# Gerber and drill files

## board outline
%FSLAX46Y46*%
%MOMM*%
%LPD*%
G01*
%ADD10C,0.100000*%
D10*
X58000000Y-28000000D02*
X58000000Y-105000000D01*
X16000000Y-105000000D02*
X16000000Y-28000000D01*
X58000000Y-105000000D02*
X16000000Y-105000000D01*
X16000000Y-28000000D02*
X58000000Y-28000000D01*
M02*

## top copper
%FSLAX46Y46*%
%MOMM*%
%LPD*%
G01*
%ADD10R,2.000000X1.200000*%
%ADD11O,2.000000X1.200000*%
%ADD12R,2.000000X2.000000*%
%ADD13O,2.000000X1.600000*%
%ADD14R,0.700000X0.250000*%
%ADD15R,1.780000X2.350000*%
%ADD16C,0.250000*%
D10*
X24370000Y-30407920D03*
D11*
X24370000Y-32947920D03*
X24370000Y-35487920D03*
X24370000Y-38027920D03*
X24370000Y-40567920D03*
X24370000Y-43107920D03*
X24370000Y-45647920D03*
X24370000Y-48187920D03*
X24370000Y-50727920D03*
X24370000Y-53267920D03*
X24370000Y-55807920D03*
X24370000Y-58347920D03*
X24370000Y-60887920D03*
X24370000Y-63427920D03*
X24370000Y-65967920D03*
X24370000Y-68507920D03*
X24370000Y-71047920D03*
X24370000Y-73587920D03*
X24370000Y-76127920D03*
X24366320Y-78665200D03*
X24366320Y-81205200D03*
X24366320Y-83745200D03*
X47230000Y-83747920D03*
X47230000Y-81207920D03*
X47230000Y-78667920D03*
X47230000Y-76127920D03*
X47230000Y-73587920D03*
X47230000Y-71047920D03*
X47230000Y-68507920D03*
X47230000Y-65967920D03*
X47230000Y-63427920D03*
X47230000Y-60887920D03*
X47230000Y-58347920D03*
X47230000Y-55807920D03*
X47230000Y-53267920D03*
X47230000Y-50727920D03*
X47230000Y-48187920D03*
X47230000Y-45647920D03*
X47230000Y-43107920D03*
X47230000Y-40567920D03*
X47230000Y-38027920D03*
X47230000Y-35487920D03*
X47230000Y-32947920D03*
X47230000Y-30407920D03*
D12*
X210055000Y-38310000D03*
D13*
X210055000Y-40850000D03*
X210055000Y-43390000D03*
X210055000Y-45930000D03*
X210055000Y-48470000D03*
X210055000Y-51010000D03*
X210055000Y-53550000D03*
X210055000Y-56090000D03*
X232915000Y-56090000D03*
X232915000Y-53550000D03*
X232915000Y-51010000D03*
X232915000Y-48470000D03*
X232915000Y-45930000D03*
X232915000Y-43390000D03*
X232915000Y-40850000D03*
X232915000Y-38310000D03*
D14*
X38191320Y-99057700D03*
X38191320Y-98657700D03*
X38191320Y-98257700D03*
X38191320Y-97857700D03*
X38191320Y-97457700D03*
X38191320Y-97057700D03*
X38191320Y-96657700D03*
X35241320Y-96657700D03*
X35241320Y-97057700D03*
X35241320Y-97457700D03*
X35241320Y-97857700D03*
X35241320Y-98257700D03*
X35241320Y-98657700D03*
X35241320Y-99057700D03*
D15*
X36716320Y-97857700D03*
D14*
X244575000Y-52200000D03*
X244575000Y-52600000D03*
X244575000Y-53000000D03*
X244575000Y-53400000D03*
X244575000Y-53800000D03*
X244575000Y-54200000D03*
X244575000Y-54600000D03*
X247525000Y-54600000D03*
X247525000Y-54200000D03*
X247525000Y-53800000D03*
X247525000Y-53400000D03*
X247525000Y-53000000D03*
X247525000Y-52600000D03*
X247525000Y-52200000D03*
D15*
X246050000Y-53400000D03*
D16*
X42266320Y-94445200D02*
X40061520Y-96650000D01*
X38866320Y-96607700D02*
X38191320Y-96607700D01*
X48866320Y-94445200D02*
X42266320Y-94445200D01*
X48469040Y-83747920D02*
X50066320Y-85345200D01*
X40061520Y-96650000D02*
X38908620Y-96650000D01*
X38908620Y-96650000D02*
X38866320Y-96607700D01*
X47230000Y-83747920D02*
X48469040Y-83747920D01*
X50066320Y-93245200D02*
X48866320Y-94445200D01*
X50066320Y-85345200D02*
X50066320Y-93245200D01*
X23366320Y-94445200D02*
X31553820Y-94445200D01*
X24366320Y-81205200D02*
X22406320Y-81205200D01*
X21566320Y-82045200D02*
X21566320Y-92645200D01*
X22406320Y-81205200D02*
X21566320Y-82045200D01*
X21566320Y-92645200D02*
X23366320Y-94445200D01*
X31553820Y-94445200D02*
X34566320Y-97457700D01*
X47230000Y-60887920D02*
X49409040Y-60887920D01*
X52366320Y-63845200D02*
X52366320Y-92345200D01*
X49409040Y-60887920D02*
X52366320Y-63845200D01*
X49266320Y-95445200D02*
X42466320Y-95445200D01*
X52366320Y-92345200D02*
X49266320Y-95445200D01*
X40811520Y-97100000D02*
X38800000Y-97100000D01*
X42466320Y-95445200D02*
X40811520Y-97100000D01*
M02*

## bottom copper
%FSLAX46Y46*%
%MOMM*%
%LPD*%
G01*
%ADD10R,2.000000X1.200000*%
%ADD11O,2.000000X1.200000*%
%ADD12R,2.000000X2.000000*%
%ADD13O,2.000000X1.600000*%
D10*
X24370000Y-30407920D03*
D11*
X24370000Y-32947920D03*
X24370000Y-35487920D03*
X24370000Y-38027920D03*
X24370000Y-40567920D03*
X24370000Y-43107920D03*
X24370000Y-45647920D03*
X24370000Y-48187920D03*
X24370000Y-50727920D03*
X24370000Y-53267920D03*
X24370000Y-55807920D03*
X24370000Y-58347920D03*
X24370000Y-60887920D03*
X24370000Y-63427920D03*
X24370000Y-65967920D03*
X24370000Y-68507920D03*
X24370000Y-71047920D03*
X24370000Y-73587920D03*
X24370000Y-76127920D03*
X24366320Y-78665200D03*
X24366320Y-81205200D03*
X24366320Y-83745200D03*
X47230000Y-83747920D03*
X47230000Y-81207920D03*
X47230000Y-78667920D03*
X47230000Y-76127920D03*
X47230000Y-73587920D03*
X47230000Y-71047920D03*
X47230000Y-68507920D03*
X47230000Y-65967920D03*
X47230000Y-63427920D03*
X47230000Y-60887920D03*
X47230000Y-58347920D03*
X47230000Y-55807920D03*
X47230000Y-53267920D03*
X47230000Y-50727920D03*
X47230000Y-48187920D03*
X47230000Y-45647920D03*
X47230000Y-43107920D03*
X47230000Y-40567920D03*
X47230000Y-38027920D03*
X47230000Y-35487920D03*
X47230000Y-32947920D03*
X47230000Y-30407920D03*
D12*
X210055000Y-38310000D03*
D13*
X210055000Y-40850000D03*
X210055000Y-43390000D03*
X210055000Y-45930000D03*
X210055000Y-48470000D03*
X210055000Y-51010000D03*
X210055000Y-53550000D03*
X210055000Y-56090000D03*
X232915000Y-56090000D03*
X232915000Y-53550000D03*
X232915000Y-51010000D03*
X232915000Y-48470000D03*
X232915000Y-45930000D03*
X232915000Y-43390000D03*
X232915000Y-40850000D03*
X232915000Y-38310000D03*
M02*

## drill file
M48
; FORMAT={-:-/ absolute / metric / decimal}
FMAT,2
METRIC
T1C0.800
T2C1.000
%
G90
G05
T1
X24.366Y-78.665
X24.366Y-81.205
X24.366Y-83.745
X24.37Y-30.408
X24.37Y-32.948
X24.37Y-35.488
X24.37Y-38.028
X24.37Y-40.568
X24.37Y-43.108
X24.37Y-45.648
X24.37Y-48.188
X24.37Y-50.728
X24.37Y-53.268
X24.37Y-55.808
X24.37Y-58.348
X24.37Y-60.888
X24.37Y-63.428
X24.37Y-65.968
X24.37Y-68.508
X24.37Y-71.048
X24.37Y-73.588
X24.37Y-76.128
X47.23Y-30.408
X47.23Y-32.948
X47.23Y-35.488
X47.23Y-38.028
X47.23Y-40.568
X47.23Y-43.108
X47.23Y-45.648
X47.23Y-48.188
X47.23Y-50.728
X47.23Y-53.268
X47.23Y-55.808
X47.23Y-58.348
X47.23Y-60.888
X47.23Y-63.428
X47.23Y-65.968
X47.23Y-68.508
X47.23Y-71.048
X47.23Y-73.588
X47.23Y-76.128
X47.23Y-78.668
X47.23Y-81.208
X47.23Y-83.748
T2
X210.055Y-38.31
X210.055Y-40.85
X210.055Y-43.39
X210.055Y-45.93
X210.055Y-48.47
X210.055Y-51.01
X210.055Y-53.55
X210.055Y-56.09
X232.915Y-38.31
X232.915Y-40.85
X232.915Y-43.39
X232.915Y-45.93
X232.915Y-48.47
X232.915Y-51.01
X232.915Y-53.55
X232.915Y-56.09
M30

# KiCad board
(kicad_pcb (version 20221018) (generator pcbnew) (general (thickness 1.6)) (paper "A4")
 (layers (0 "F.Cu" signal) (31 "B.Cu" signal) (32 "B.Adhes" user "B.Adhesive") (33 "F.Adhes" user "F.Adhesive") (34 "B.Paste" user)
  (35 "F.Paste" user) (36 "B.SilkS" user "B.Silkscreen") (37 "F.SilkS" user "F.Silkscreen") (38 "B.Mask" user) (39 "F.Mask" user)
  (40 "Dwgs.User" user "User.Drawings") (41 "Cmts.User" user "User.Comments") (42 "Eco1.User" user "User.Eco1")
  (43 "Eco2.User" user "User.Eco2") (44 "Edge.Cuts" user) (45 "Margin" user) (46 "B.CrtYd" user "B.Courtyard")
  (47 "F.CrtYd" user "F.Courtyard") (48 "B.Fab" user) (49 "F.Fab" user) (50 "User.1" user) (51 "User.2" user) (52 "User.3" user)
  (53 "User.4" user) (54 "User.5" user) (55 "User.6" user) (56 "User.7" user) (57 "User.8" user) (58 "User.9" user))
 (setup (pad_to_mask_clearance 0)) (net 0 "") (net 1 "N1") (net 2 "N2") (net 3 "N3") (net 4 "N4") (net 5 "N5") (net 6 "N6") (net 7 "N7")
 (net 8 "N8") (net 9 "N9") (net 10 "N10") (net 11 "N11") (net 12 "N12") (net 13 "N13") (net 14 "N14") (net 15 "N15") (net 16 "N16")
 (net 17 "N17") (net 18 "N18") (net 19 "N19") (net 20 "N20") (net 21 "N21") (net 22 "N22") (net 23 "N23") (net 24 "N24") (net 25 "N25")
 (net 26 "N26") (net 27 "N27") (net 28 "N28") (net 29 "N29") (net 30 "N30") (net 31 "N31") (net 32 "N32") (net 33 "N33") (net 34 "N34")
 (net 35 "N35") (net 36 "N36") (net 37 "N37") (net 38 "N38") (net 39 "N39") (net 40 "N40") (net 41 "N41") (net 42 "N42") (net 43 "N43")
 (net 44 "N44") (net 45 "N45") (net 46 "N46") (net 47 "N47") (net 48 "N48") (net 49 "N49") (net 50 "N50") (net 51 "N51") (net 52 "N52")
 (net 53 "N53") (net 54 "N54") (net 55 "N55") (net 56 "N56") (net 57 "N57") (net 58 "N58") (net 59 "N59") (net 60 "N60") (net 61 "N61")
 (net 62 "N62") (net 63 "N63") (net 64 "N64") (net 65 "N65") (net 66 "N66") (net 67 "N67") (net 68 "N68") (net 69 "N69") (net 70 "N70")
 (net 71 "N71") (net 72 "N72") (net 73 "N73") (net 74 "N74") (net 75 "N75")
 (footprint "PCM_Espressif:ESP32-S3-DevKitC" (layer "F.Cu") (at 24.37 30.40792)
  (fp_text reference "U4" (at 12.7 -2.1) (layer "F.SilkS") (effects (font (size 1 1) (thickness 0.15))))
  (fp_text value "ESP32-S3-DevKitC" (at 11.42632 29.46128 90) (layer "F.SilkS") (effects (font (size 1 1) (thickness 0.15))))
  (pad "1" thru_hole rect (at 0 0 270) (size 1.2 2) (drill 0.8) (layers "*.Cu" "*.Mask") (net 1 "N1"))
  (pad "2" thru_hole oval (at 0 2.54 270) (size 1.2 2) (drill 0.8) (layers "*.Cu" "*.Mask") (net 1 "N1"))
  (pad "3" thru_hole oval (at 0 5.08 270) (size 1.2 2) (drill 0.8) (layers "*.Cu" "*.Mask") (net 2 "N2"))
  (pad "4" thru_hole oval (at 0 7.62 270) (size 1.2 2) (drill 0.8) (layers "*.Cu" "*.Mask") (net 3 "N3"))
  (pad "5" thru_hole oval (at 0 10.16 270) (size 1.2 2) (drill 0.8) (layers "*.Cu" "*.Mask") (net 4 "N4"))
  (pad "6" thru_hole oval (at 0 12.7 270) (size 1.2 2) (drill 0.8) (layers "*.Cu" "*.Mask") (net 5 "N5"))
  (pad "7" thru_hole oval (at 0 15.24 270) (size 1.2 2) (drill 0.8) (layers "*.Cu" "*.Mask") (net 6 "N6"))
  (pad "8" thru_hole oval (at 0 17.78 270) (size 1.2 2) (drill 0.8) (layers "*.Cu" "*.Mask") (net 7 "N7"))
  (pad "9" thru_hole oval (at 0 20.32 270) (size 1.2 2) (drill 0.8) (layers "*.Cu" "*.Mask") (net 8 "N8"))
  (pad "10" thru_hole oval (at 0 22.86 270) (size 1.2 2) (drill 0.8) (layers "*.Cu" "*.Mask") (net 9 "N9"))
  (pad "11" thru_hole oval (at 0 25.4 270) (size 1.2 2) (drill 0.8) (layers "*.Cu" "*.Mask") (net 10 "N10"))
  (pad "12" thru_hole oval (at 0 27.94 270) (size 1.2 2) (drill 0.8) (layers "*.Cu" "*.Mask") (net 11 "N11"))
  (pad "13" thru_hole oval (at 0 30.48 270) (size 1.2 2) (drill 0.8) (layers "*.Cu" "*.Mask") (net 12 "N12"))
  (pad "14" thru_hole oval (at 0 33.02 270) (size 1.2 2) (drill 0.8) (layers "*.Cu" "*.Mask") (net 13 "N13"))
  (pad "15" thru_hole oval (at 0 35.56 270) (size 1.2 2) (drill 0.8) (layers "*.Cu" "*.Mask") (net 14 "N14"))
  (pad "16" thru_hole oval (at 0 38.1 270) (size 1.2 2) (drill 0.8) (layers "*.Cu" "*.Mask") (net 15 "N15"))
  (pad "17" thru_hole oval (at 0 40.64 270) (size 1.2 2) (drill 0.8) (layers "*.Cu" "*.Mask") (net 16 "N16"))
  (pad "18" thru_hole oval (at 0 43.18 270) (size 1.2 2) (drill 0.8) (layers "*.Cu" "*.Mask") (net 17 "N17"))
  (pad "19" thru_hole oval (at 0 45.72 270) (size 1.2 2) (drill 0.8) (layers "*.Cu" "*.Mask") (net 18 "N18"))
  (pad "20" thru_hole oval (at -0.00368 48.25728 270) (size 1.2 2) (drill 0.8) (layers "*.Cu" "*.Mask") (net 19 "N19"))
  (pad "21" thru_hole oval (at -0.00368 50.79728 270) (size 1.2 2) (drill 0.8) (layers "*.Cu" "*.Mask") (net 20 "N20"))
  (pad "22" thru_hole oval (at -0.00368 53.33728 270) (size 1.2 2) (drill 0.8) (layers "*.Cu" "*.Mask") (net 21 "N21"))
  (pad "23" thru_hole oval (at 22.86 53.34 270) (size 1.2 2) (drill 0.8) (layers "*.Cu" "*.Mask") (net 21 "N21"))
  (pad "24" thru_hole oval (at 22.86 50.8 270) (size 1.2 2) (drill 0.8) (layers "*.Cu" "*.Mask") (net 21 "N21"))
  (pad "25" thru_hole oval (at 22.86 48.26 270) (size 1.2 2) (drill 0.8) (layers "*.Cu" "*.Mask") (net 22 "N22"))
  (pad "26" thru_hole oval (at 22.86 45.72 270) (size 1.2 2) (drill 0.8) (layers "*.Cu" "*.Mask") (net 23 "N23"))
  (pad "27" thru_hole oval (at 22.86 43.18 270) (size 1.2 2) (drill 0.8) (layers "*.Cu" "*.Mask") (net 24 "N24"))
  (pad "28" thru_hole oval (at 22.86 40.64 270) (size 1.2 2) (drill 0.8) (layers "*.Cu" "*.Mask") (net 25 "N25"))
  (pad "29" thru_hole oval (at 22.86 38.1 270) (size 1.2 2) (drill 0.8) (layers "*.Cu" "*.Mask") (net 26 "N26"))
  (pad "30" thru_hole oval (at 22.86 35.56 270) (size 1.2 2) (drill 0.8) (layers "*.Cu" "*.Mask") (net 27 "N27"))
  (pad "31" thru_hole oval (at 22.86 33.02 270) (size 1.2 2) (drill 0.8) (layers "*.Cu" "*.Mask") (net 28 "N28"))
  (pad "32" thru_hole oval (at 22.86 30.48 270) (size 1.2 2) (drill 0.8) (layers "*.Cu" "*.Mask") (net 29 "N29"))
  (pad "33" thru_hole oval (at 22.86 27.94 270) (size 1.2 2) (drill 0.8) (layers "*.Cu" "*.Mask") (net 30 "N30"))
  (pad "34" thru_hole oval (at 22.86 25.4 270) (size 1.2 2) (drill 0.8) (layers "*.Cu" "*.Mask") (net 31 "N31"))
  (pad "35" thru_hole oval (at 22.86 22.86 270) (size 1.2 2) (drill 0.8) (layers "*.Cu" "*.Mask") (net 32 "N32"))
  (pad "36" thru_hole oval (at 22.86 20.32 270) (size 1.2 2) (drill 0.8) (layers "*.Cu" "*.Mask") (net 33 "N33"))
  (pad "37" thru_hole oval (at 22.86 17.78 270) (size 1.2 2) (drill 0.8) (layers "*.Cu" "*.Mask") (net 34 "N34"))
  (pad "38" thru_hole oval (at 22.86 15.24 270) (size 1.2 2) (drill 0.8) (layers "*.Cu" "*.Mask") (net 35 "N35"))
  (pad "39" thru_hole oval (at 22.86 12.7 270) (size 1.2 2) (drill 0.8) (layers "*.Cu" "*.Mask") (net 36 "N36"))
  (pad "40" thru_hole oval (at 22.86 10.16 270) (size 1.2 2) (drill 0.8) (layers "*.Cu" "*.Mask") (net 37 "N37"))
  (pad "41" thru_hole oval (at 22.86 7.62 270) (size 1.2 2) (drill 0.8) (layers "*.Cu" "*.Mask") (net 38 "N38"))
  (pad "42" thru_hole oval (at 22.86 5.08 270) (size 1.2 2) (drill 0.8) (layers "*.Cu" "*.Mask") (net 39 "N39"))
  (pad "43" thru_hole oval (at 22.86 2.54 270) (size 1.2 2) (drill 0.8) (layers "*.Cu" "*.Mask") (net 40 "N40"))
  (pad "44" thru_hole oval (at 22.86 0 270) (size 1.2 2) (drill 0.8) (layers "*.Cu" "*.Mask") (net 21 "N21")))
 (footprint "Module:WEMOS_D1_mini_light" (layer "F.Cu") (at 210.055 38.31)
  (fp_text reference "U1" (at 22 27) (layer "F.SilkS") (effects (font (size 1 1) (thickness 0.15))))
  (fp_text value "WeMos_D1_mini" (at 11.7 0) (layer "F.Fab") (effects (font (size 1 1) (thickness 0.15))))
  (pad "1" thru_hole rect (at 0 0) (size 2 2) (drill 1) (layers "*.Cu" "*.Mask") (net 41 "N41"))
  (pad "2" thru_hole oval (at 0 2.54) (size 2 1.6) (drill 1) (layers "*.Cu" "*.Mask") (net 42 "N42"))
  (pad "3" thru_hole oval (at 0 5.08) (size 2 1.6) (drill 1) (layers "*.Cu" "*.Mask") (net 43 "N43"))
  (pad "4" thru_hole oval (at 0 7.62) (size 2 1.6) (drill 1) (layers "*.Cu" "*.Mask") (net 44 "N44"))
  (pad "5" thru_hole oval (at 0 10.16) (size 2 1.6) (drill 1) (layers "*.Cu" "*.Mask") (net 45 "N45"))
  (pad "6" thru_hole oval (at 0 12.7) (size 2 1.6) (drill 1) (layers "*.Cu" "*.Mask") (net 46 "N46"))
  (pad "7" thru_hole oval (at 0 15.24) (size 2 1.6) (drill 1) (layers "*.Cu" "*.Mask") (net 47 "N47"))
  (pad "8" thru_hole oval (at 0 17.78) (size 2 1.6) (drill 1) (layers "*.Cu" "*.Mask") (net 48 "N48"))
  (pad "9" thru_hole oval (at 22.86 17.78) (size 2 1.6) (drill 1) (layers "*.Cu" "*.Mask") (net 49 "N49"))
  (pad "10" thru_hole oval (at 22.86 15.24) (size 2 1.6) (drill 1) (layers "*.Cu" "*.Mask") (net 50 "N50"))
  (pad "11" thru_hole oval (at 22.86 12.7) (size 2 1.6) (drill 1) (layers "*.Cu" "*.Mask") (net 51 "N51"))
  (pad "12" thru_hole oval (at 22.86 10.16) (size 2 1.6) (drill 1) (layers "*.Cu" "*.Mask") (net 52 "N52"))
  (pad "13" thru_hole oval (at 22.86 7.62) (size 2 1.6) (drill 1) (layers "*.Cu" "*.Mask") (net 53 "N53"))
  (pad "14" thru_hole oval (at 22.86 5.08) (size 2 1.6) (drill 1) (layers "*.Cu" "*.Mask") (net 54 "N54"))
  (pad "15" thru_hole oval (at 22.86 2.54) (size 2 1.6) (drill 1) (layers "*.Cu" "*.Mask") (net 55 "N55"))
  (pad "16" thru_hole oval (at 22.86 0) (size 2 1.6) (drill 1) (layers "*.Cu" "*.Mask") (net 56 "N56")))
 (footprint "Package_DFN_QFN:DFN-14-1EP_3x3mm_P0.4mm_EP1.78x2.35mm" (layer "F.Cu") (at 36.71632 97.8577 180)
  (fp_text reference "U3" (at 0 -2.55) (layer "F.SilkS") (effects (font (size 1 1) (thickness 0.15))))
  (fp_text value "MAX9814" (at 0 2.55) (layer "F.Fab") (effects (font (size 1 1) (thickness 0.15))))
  (pad "" smd rect (at -0.445 -0.5875 180) (size 0.7 0.97) (layers "F.Paste"))
  (pad "" smd rect (at -0.445 0.5875 180) (size 0.7 0.97) (layers "F.Paste"))
  (pad "" smd rect (at 0.45 -0.5875 180) (size 0.7 0.97) (layers "F.Paste"))
  (pad "" smd rect (at 0.45 0.5875 180) (size 0.7 0.97) (layers "F.Paste"))
  (pad "1" smd rect (at -1.475 -1.2 180) (size 0.7 0.25) (layers "F.Cu" "F.Paste" "F.Mask") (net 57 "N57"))
  (pad "2" smd rect (at -1.475 -0.8 180) (size 0.7 0.25) (layers "F.Cu" "F.Paste" "F.Mask") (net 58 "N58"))
  (pad "3" smd rect (at -1.475 -0.4 180) (size 0.7 0.25) (layers "F.Cu" "F.Paste" "F.Mask") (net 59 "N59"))
  (pad "4" smd rect (at -1.475 0 180) (size 0.7 0.25) (layers "F.Cu" "F.Paste" "F.Mask") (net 21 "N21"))
  (pad "5" smd rect (at -1.475 0.4 180) (size 0.7 0.25) (layers "F.Cu" "F.Paste" "F.Mask") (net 20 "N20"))
  (pad "6" smd rect (at -1.475 0.8 180) (size 0.7 0.25) (layers "F.Cu" "F.Paste" "F.Mask") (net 29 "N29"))
  (pad "7" smd rect (at -1.475 1.2 180) (size 0.7 0.25) (layers "F.Cu" "F.Paste" "F.Mask") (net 21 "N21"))
  (pad "8" smd rect (at 1.475 1.2 180) (size 0.7 0.25) (layers "F.Cu" "F.Paste" "F.Mask") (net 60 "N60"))
  (pad "9" smd rect (at 1.475 0.8 180) (size 0.7 0.25) (layers "F.Cu" "F.Paste" "F.Mask") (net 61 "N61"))
  (pad "10" smd rect (at 1.475 0.4 180) (size 0.7 0.25) (layers "F.Cu" "F.Paste" "F.Mask") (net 20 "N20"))
  (pad "11" smd rect (at 1.475 0 180) (size 0.7 0.25) (layers "F.Cu" "F.Paste" "F.Mask") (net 21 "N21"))
  (pad "12" smd rect (at 1.475 -0.4 180) (size 0.7 0.25) (layers "F.Cu" "F.Paste" "F.Mask") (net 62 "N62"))
  (pad "13" smd rect (at 1.475 -0.8 180) (size 0.7 0.25) (layers "F.Cu" "F.Paste" "F.Mask") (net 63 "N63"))
  (pad "14" smd rect (at 1.475 -1.2 180) (size 0.7 0.25) (layers "F.Cu" "F.Paste" "F.Mask") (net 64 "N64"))
  (pad "15" smd rect (at 0 0 180) (size 1.78 2.35) (layers "F.Cu" "F.Mask") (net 21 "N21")))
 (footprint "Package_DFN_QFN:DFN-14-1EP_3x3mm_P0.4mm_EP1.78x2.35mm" (layer "F.Cu") (at 246.05 53.4)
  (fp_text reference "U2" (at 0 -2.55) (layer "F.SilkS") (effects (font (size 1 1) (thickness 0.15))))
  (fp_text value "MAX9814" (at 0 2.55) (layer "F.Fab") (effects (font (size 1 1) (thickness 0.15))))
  (pad "" smd rect (at -0.445 -0.5875) (size 0.7 0.97) (layers "F.Paste"))
  (pad "" smd rect (at -0.445 0.5875) (size 0.7 0.97) (layers "F.Paste"))
  (pad "" smd rect (at 0.45 -0.5875) (size 0.7 0.97) (layers "F.Paste"))
  (pad "" smd rect (at 0.45 0.5875) (size 0.7 0.97) (layers "F.Paste"))
  (pad "1" smd rect (at -1.475 -1.2) (size 0.7 0.25) (layers "F.Cu" "F.Paste" "F.Mask") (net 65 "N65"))
  (pad "2" smd rect (at -1.475 -0.8) (size 0.7 0.25) (layers "F.Cu" "F.Paste" "F.Mask") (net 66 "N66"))
  (pad "3" smd rect (at -1.475 -0.4) (size 0.7 0.25) (layers "F.Cu" "F.Paste" "F.Mask") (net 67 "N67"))
  (pad "4" smd rect (at -1.475 0) (size 0.7 0.25) (layers "F.Cu" "F.Paste" "F.Mask") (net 50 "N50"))
  (pad "5" smd rect (at -1.475 0.4) (size 0.7 0.25) (layers "F.Cu" "F.Paste" "F.Mask") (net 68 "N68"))
  (pad "6" smd rect (at -1.475 0.8) (size 0.7 0.25) (layers "F.Cu" "F.Paste" "F.Mask") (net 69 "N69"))
  (pad "7" smd rect (at -1.475 1.2) (size 0.7 0.25) (layers "F.Cu" "F.Paste" "F.Mask") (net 50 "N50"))
  (pad "8" smd rect (at 1.475 1.2) (size 0.7 0.25) (layers "F.Cu" "F.Paste" "F.Mask") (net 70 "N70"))
  (pad "9" smd rect (at 1.475 0.8) (size 0.7 0.25) (layers "F.Cu" "F.Paste" "F.Mask") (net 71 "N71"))
  (pad "10" smd rect (at 1.475 0.4) (size 0.7 0.25) (layers "F.Cu" "F.Paste" "F.Mask") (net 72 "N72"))
  (pad "11" smd rect (at 1.475 0) (size 0.7 0.25) (layers "F.Cu" "F.Paste" "F.Mask") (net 50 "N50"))
  (pad "12" smd rect (at 1.475 -0.4) (size 0.7 0.25) (layers "F.Cu" "F.Paste" "F.Mask") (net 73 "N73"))
  (pad "13" smd rect (at 1.475 -0.8) (size 0.7 0.25) (layers "F.Cu" "F.Paste" "F.Mask") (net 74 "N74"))
  (pad "14" smd rect (at 1.475 -1.2) (size 0.7 0.25) (layers "F.Cu" "F.Paste" "F.Mask") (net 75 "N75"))
  (pad "15" smd rect (at 0 0) (size 1.78 2.35) (layers "F.Cu" "F.Mask") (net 50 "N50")))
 (gr_line (start 58 28) (end 58 105) (stroke (width 0.1) (type default)) (layer "Edge.Cuts"))
 (gr_line (start 16 105) (end 16 28) (stroke (width 0.1) (type default)) (layer "Edge.Cuts"))
 (gr_line (start 58 105) (end 16 105) (stroke (width 0.1) (type default)) (layer "Edge.Cuts"))
 (gr_line (start 16 28) (end 58 28) (stroke (width 0.1) (type default)) (layer "Edge.Cuts"))
 (segment (start 42.26632 94.4452) (end 40.06152 96.65) (width 0.25) (layer "F.Cu") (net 21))
 (segment (start 38.86632 96.6077) (end 38.19132 96.6077) (width 0.25) (layer "F.Cu") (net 21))
 (segment (start 48.86632 94.4452) (end 42.26632 94.4452) (width 0.25) (layer "F.Cu") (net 21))
 (segment (start 48.46904 83.74792) (end 50.06632 85.3452) (width 0.25) (layer "F.Cu") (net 21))
 (segment (start 40.06152 96.65) (end 38.90862 96.65) (width 0.25) (layer "F.Cu") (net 21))
 (segment (start 38.90862 96.65) (end 38.86632 96.6077) (width 0.25) (layer "F.Cu") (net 21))
 (segment (start 47.23 83.74792) (end 48.46904 83.74792) (width 0.25) (layer "F.Cu") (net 21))
 (segment (start 50.06632 93.2452) (end 48.86632 94.4452) (width 0.25) (layer "F.Cu") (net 21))
 (segment (start 50.06632 85.3452) (end 50.06632 93.2452) (width 0.25) (layer "F.Cu") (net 21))
 (segment (start 23.36632 94.4452) (end 31.55382 94.4452) (width 0.25) (layer "F.Cu") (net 20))
 (segment (start 24.36632 81.2052) (end 22.40632 81.2052) (width 0.25) (layer "F.Cu") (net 20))
 (segment (start 21.56632 82.0452) (end 21.56632 92.6452) (width 0.25) (layer "F.Cu") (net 20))
 (segment (start 22.40632 81.2052) (end 21.56632 82.0452) (width 0.25) (layer "F.Cu") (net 20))
 (segment (start 21.56632 92.6452) (end 23.36632 94.4452) (width 0.25) (layer "F.Cu") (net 20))
 (segment (start 31.55382 94.4452) (end 34.56632 97.4577) (width 0.25) (layer "F.Cu") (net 20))
 (segment (start 47.23 60.88792) (end 49.40904 60.88792) (width 0.25) (layer "F.Cu") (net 29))
 (segment (start 52.36632 63.8452) (end 52.36632 92.3452) (width 0.25) (layer "F.Cu") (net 29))
 (segment (start 49.40904 60.88792) (end 52.36632 63.8452) (width 0.25) (layer "F.Cu") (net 29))
 (segment (start 49.26632 95.4452) (end 42.46632 95.4452) (width 0.25) (layer "F.Cu") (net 29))
 (segment (start 52.36632 92.3452) (end 49.26632 95.4452) (width 0.25) (layer "F.Cu") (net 29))
 (segment (start 40.81152 97.1) (end 38.8 97.1) (width 0.25) (layer "F.Cu") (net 29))
 (segment (start 42.46632 95.4452) (end 40.81152 97.1) (width 0.25) (layer "F.Cu") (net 29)))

